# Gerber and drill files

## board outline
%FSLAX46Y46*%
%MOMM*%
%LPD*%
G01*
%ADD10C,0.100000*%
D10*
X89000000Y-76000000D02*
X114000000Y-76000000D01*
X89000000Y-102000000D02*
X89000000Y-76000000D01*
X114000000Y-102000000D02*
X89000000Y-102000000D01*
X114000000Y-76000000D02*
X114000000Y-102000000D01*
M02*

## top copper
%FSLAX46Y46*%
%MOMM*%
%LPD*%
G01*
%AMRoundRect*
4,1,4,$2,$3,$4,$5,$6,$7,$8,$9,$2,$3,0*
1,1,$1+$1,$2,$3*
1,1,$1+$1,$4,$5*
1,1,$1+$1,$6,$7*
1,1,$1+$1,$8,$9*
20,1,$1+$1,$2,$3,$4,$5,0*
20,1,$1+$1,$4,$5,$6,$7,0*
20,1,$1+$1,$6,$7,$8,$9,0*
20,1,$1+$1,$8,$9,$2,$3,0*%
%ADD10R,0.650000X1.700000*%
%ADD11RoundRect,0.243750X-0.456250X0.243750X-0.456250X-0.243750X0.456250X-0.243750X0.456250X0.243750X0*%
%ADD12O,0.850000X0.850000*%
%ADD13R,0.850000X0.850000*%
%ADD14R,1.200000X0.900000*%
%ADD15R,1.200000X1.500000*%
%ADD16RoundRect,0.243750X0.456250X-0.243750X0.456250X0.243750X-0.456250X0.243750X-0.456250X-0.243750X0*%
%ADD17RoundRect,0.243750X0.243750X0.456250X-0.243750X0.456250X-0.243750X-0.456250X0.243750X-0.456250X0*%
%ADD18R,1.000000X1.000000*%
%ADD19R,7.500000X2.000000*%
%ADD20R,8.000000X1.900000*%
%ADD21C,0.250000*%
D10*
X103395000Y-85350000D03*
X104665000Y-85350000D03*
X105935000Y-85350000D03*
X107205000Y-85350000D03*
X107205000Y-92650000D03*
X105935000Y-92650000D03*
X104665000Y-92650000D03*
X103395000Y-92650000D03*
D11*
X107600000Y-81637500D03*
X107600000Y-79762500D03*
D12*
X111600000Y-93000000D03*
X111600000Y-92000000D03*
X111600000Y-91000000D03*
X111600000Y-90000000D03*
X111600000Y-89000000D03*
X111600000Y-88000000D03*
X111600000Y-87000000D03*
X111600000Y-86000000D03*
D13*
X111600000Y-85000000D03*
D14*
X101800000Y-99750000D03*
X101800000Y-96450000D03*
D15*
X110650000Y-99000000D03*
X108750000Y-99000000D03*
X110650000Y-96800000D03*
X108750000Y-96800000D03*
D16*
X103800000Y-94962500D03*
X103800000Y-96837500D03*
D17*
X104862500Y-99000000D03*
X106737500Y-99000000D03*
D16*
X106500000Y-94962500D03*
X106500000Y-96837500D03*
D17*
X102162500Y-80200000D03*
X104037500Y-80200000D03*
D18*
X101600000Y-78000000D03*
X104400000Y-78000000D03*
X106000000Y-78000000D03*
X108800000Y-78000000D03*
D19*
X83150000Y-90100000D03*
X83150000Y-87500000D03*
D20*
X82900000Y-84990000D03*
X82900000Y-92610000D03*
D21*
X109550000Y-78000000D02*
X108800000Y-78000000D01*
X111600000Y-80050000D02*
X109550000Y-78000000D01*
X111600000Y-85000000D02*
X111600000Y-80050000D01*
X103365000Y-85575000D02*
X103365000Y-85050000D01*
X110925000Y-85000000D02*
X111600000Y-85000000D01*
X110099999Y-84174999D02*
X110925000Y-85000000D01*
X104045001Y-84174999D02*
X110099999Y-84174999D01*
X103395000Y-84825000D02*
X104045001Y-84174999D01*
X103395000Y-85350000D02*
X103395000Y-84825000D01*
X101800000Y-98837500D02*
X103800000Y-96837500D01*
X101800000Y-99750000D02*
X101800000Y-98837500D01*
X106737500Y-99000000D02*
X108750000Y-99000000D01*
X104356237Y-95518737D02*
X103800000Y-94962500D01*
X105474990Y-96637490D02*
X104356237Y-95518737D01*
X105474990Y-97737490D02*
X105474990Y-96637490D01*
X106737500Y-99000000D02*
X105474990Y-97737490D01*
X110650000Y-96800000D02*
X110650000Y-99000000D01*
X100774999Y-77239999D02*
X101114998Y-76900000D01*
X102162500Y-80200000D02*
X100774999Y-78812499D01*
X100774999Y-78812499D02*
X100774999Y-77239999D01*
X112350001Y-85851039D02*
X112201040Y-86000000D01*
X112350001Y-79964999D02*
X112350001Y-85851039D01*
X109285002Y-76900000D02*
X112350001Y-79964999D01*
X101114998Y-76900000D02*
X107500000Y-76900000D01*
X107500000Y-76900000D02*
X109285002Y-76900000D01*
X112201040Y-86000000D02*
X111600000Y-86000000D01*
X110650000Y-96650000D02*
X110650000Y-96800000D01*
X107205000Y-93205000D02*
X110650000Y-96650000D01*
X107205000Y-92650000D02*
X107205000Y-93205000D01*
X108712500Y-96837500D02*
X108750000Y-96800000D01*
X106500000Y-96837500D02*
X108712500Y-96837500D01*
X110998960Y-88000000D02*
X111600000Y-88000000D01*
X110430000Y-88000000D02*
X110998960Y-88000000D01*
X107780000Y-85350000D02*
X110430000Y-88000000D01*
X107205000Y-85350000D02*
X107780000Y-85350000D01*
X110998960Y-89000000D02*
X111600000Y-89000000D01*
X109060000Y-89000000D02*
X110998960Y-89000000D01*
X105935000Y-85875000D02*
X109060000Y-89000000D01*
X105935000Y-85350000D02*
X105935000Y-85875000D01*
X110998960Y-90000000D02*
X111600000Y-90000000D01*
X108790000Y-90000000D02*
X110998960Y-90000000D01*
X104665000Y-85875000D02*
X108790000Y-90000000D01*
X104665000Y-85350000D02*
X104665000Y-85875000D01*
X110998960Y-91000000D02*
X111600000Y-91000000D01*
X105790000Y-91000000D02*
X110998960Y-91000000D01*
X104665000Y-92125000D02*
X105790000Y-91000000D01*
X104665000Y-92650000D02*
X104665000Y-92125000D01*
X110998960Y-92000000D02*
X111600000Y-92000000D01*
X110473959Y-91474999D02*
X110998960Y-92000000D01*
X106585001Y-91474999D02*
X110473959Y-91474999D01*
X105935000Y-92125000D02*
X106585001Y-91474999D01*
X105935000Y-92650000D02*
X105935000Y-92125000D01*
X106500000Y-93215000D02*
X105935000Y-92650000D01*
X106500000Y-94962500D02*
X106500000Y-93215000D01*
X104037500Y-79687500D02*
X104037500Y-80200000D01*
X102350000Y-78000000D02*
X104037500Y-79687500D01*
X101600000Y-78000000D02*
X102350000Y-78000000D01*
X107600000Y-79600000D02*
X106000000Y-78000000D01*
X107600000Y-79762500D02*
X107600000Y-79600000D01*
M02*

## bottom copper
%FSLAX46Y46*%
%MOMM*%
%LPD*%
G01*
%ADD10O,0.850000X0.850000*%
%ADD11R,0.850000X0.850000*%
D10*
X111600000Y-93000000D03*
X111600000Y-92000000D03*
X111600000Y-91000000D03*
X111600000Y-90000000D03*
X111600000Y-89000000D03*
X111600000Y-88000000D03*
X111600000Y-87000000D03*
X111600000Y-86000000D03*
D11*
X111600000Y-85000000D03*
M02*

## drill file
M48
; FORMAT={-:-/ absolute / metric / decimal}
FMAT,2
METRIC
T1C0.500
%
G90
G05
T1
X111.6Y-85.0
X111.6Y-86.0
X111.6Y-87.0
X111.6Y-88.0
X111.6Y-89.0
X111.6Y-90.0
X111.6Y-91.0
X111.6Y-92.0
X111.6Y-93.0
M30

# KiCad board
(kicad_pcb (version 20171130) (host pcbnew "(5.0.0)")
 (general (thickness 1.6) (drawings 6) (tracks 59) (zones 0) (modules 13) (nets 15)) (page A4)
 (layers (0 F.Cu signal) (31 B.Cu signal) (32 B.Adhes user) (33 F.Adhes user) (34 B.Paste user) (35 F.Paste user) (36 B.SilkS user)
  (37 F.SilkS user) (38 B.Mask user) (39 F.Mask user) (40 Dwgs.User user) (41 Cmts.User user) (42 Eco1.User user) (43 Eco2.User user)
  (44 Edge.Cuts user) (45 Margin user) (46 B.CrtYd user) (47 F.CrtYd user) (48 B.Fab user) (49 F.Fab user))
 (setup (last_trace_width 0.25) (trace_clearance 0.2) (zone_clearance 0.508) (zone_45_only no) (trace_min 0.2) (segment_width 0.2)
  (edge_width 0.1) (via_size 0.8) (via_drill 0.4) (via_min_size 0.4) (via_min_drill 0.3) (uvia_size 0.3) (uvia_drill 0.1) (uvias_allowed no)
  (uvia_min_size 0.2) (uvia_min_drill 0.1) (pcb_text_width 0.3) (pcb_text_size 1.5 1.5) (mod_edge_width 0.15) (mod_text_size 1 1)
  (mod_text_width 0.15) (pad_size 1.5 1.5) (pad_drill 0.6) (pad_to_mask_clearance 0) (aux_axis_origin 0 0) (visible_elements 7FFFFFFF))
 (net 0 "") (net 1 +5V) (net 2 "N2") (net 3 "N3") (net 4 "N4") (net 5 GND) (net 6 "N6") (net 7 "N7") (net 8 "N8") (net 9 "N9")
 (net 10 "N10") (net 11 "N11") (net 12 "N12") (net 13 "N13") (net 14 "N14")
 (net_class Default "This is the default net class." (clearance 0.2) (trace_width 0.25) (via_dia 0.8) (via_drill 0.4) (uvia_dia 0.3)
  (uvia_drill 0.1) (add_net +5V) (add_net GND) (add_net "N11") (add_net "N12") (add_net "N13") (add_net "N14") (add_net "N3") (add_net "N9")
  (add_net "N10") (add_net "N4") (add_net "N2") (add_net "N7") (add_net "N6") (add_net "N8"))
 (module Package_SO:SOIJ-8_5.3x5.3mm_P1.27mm (layer F.Cu) (at 105.3 89 90)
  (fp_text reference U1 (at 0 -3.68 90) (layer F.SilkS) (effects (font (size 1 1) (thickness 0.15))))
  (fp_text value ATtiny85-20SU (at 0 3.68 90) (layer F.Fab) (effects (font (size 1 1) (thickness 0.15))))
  (pad 8 smd rect (at 3.65 -1.905 90) (size 1.7 0.65) (layers F.Cu F.Paste F.Mask) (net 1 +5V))
  (pad 7 smd rect (at 3.65 -0.635 90) (size 1.7 0.65) (layers F.Cu F.Paste F.Mask) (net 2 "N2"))
  (pad 6 smd rect (at 3.65 0.635 90) (size 1.7 0.65) (layers F.Cu F.Paste F.Mask) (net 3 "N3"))
  (pad 5 smd rect (at 3.65 1.905 90) (size 1.7 0.65) (layers F.Cu F.Paste F.Mask) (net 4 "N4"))
  (pad 4 smd rect (at -3.65 1.905 90) (size 1.7 0.65) (layers F.Cu F.Paste F.Mask) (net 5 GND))
  (pad 3 smd rect (at -3.65 0.635 90) (size 1.7 0.65) (layers F.Cu F.Paste F.Mask) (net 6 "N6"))
  (pad 2 smd rect (at -3.65 -0.635 90) (size 1.7 0.65) (layers F.Cu F.Paste F.Mask) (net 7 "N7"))
  (pad 1 smd rect (at -3.65 -1.905 90) (size 1.7 0.65) (layers F.Cu F.Paste F.Mask) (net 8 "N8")))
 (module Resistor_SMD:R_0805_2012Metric (layer F.Cu) (at 107.6 80.7 270)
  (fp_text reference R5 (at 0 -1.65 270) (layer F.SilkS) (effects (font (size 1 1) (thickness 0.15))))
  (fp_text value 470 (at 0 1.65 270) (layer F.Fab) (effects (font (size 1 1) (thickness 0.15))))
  (pad 2 smd roundrect (at 0.9375 0 270) (size 0.975 1.4) (layers F.Cu F.Paste F.Mask) (roundrect_rratio 0.25) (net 5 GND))
  (pad 1 smd roundrect (at -0.9375 0 270) (size 0.975 1.4) (layers F.Cu F.Paste F.Mask) (roundrect_rratio 0.25) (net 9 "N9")))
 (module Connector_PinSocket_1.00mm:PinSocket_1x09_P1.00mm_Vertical (layer F.Cu) (at 111.6 85)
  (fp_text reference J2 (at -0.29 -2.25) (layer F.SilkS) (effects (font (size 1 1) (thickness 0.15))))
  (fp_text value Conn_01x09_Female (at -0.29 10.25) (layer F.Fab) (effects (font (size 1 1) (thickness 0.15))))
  (pad 9 thru_hole oval (at 0 8) (size 0.85 0.85) (drill 0.5) (layers *.Cu *.Mask) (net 8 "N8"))
  (pad 8 thru_hole oval (at 0 7) (size 0.85 0.85) (drill 0.5) (layers *.Cu *.Mask) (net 6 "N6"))
  (pad 7 thru_hole oval (at 0 6) (size 0.85 0.85) (drill 0.5) (layers *.Cu *.Mask) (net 7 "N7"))
  (pad 6 thru_hole oval (at 0 5) (size 0.85 0.85) (drill 0.5) (layers *.Cu *.Mask) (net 2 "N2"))
  (pad 5 thru_hole oval (at 0 4) (size 0.85 0.85) (drill 0.5) (layers *.Cu *.Mask) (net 3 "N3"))
  (pad 4 thru_hole oval (at 0 3) (size 0.85 0.85) (drill 0.5) (layers *.Cu *.Mask) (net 4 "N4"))
  (pad 3 thru_hole oval (at 0 2) (size 0.85 0.85) (drill 0.5) (layers *.Cu *.Mask) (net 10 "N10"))
  (pad 2 thru_hole oval (at 0 1) (size 0.85 0.85) (drill 0.5) (layers *.Cu *.Mask) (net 5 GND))
  (pad 1 thru_hole rect (at 0 0) (size 0.85 0.85) (drill 0.5) (layers *.Cu *.Mask) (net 1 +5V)))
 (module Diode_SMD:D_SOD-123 (layer F.Cu) (at 101.8 98.1 270)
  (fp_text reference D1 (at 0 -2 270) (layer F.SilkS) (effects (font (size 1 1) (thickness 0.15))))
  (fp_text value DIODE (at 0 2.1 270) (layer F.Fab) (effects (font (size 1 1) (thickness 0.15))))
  (pad 2 smd rect (at 1.65 0 270) (size 0.9 1.2) (layers F.Cu F.Paste F.Mask) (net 1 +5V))
  (pad 1 smd rect (at -1.65 0 270) (size 0.9 1.2) (layers F.Cu F.Paste F.Mask) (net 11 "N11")))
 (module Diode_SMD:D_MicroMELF (layer F.Cu) (at 109.7 99)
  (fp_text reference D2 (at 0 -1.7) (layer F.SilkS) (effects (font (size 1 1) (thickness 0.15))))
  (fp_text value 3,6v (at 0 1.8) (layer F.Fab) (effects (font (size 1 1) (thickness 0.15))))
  (pad 2 smd rect (at 0.95 0) (size 1.2 1.5) (layers F.Cu F.Paste F.Mask) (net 5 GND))
  (pad 1 smd rect (at -0.95 0) (size 1.2 1.5) (layers F.Cu F.Paste F.Mask) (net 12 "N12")))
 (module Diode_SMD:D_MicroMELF (layer F.Cu) (at 109.7 96.8)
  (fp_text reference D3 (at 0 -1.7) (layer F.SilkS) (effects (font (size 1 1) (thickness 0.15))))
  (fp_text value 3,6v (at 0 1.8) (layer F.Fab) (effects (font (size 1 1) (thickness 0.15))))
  (pad 2 smd rect (at 0.95 0) (size 1.2 1.5) (layers F.Cu F.Paste F.Mask) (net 5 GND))
  (pad 1 smd rect (at -0.95 0) (size 1.2 1.5) (layers F.Cu F.Paste F.Mask) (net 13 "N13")))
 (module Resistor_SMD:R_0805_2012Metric (layer F.Cu) (at 103.8 95.9 90)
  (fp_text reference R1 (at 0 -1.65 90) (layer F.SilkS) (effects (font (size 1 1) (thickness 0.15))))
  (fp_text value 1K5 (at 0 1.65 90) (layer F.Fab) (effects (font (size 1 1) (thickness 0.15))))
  (pad 2 smd roundrect (at 0.9375 0 90) (size 0.975 1.4) (layers F.Cu F.Paste F.Mask) (roundrect_rratio 0.25) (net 12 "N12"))
  (pad 1 smd roundrect (at -0.9375 0 90) (size 0.975 1.4) (layers F.Cu F.Paste F.Mask) (roundrect_rratio 0.25) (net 1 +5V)))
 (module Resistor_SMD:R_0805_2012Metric (layer F.Cu) (at 105.8 99 180)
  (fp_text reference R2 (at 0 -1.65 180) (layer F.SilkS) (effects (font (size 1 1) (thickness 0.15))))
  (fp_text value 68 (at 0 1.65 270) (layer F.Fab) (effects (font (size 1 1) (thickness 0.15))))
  (pad 2 smd roundrect (at 0.9375 0 180) (size 0.975 1.4) (layers F.Cu F.Paste F.Mask) (roundrect_rratio 0.25) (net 7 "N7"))
  (pad 1 smd roundrect (at -0.9375 0 180) (size 0.975 1.4) (layers F.Cu F.Paste F.Mask) (roundrect_rratio 0.25) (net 12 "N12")))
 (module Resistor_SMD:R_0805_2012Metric (layer F.Cu) (at 106.5 95.9 90)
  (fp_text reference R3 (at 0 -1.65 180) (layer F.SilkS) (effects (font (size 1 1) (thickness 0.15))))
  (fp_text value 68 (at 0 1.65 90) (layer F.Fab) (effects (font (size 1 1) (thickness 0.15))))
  (pad 2 smd roundrect (at 0.9375 0 90) (size 0.975 1.4) (layers F.Cu F.Paste F.Mask) (roundrect_rratio 0.25) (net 6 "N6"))
  (pad 1 smd roundrect (at -0.9375 0 90) (size 0.975 1.4) (layers F.Cu F.Paste F.Mask) (roundrect_rratio 0.25) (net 13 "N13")))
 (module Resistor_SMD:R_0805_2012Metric (layer F.Cu) (at 103.1 80.2 180)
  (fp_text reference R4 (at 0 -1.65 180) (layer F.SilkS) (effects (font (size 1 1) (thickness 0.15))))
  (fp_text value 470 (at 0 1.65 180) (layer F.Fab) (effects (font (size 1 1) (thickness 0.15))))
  (pad 2 smd roundrect (at 0.9375 0 180) (size 0.975 1.4) (layers F.Cu F.Paste F.Mask) (roundrect_rratio 0.25) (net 5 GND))
  (pad 1 smd roundrect (at -0.9375 0 180) (size 0.975 1.4) (layers F.Cu F.Paste F.Mask) (roundrect_rratio 0.25) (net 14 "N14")))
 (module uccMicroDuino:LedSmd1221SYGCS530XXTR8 (layer F.Cu) (at 103 78)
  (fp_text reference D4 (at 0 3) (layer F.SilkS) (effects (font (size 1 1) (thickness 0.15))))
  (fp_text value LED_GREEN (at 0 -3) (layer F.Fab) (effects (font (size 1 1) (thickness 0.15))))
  (pad 1 smd rect (at -1.4 0) (size 1 1) (layers F.Cu F.Paste F.Mask) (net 14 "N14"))
  (pad 2 smd rect (at 1.4 0) (size 1 1) (layers F.Cu F.Paste F.Mask) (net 3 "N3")))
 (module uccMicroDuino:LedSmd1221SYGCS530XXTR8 (layer F.Cu) (at 107.4 78)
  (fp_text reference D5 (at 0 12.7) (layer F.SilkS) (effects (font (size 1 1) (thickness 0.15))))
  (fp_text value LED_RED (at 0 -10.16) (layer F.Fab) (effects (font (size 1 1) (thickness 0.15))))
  (pad 1 smd rect (at -1.4 0) (size 1 1) (layers F.Cu F.Paste F.Mask) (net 9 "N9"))
  (pad 2 smd rect (at 1.4 0) (size 1 1) (layers F.Cu F.Paste F.Mask) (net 1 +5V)))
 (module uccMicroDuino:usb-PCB (layer F.Cu) (at 78 88.8 270)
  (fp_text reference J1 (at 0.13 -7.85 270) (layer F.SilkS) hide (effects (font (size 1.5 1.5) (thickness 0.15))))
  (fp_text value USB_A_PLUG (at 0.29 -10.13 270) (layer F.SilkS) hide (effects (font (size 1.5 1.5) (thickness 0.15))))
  (pad 2 connect rect (at 1.3 -5.15 270) (size 2 7.5) (layers F.Cu F.Mask) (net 12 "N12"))
  (pad 3 connect rect (at -1.3 -5.15 270) (size 2 7.5) (layers F.Cu F.Mask) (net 13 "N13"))
  (pad 4 connect rect (at -3.81 -4.9 270) (size 1.9 8) (layers F.Cu F.Mask) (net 5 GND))
  (pad 1 connect rect (at 3.81 -4.9 270) (size 1.9 8) (layers F.Cu F.Mask) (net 11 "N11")))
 (gr_line (start 89 76) (end 114 76) (layer Edge.Cuts) (width 0.1))
 (gr_line (start 89 102) (end 89 76) (layer Edge.Cuts) (width 0.1))
 (gr_line (start 114 102) (end 89 102) (layer Edge.Cuts) (width 0.1))
 (gr_line (start 114 76) (end 114 102) (layer Edge.Cuts) (width 0.1))
 (segment (start 109.55 78) (end 108.8 78) (width 0.25) (layer F.Cu) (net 1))
 (segment (start 111.6 80.05) (end 109.55 78) (width 0.25) (layer F.Cu) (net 1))
 (segment (start 111.6 85) (end 111.6 80.05) (width 0.25) (layer F.Cu) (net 1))
 (segment (start 103.365 85.575) (end 103.365 85.05) (width 0.25) (layer F.Cu) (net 1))
 (segment (start 110.925 85) (end 111.6 85) (width 0.25) (layer F.Cu) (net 1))
 (segment (start 110.099999 84.174999) (end 110.925 85) (width 0.25) (layer F.Cu) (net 1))
 (segment (start 104.045001 84.174999) (end 110.099999 84.174999) (width 0.25) (layer F.Cu) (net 1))
 (segment (start 103.395 84.825) (end 104.045001 84.174999) (width 0.25) (layer F.Cu) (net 1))
 (segment (start 103.395 85.35) (end 103.395 84.825) (width 0.25) (layer F.Cu) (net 1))
 (segment (start 101.8 98.8375) (end 103.8 96.8375) (width 0.25) (layer F.Cu) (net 1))
 (segment (start 101.8 99.75) (end 101.8 98.8375) (width 0.25) (layer F.Cu) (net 1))
 (segment (start 106.7375 99) (end 108.75 99) (width 0.25) (layer F.Cu) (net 12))
 (segment (start 104.356237 95.518737) (end 103.8 94.9625) (width 0.25) (layer F.Cu) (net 12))
 (segment (start 105.47499 96.63749) (end 104.356237 95.518737) (width 0.25) (layer F.Cu) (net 12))
 (segment (start 105.47499 97.73749) (end 105.47499 96.63749) (width 0.25) (layer F.Cu) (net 12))
 (segment (start 106.7375 99) (end 105.47499 97.73749) (width 0.25) (layer F.Cu) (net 12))
 (segment (start 110.65 96.8) (end 110.65 99) (width 0.25) (layer F.Cu) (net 5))
 (segment (start 100.774999 77.239999) (end 101.114998 76.9) (width 0.25) (layer F.Cu) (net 5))
 (segment (start 102.1625 80.2) (end 100.774999 78.812499) (width 0.25) (layer F.Cu) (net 5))
 (segment (start 100.774999 78.812499) (end 100.774999 77.239999) (width 0.25) (layer F.Cu) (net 5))
 (segment (start 112.350001 85.851039) (end 112.20104 86) (width 0.25) (layer F.Cu) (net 5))
 (segment (start 112.350001 79.964999) (end 112.350001 85.851039) (width 0.25) (layer F.Cu) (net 5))
 (segment (start 109.285002 76.9) (end 112.350001 79.964999) (width 0.25) (layer F.Cu) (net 5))
 (segment (start 101.114998 76.9) (end 107.5 76.9) (width 0.25) (layer F.Cu) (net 5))
 (segment (start 107.5 76.9) (end 109.285002 76.9) (width 0.25) (layer F.Cu) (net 5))
 (segment (start 112.20104 86) (end 111.6 86) (width 0.25) (layer F.Cu) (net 5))
 (segment (start 110.65 96.65) (end 110.65 96.8) (width 0.25) (layer F.Cu) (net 5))
 (segment (start 107.205 93.205) (end 110.65 96.65) (width 0.25) (layer F.Cu) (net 5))
 (segment (start 107.205 92.65) (end 107.205 93.205) (width 0.25) (layer F.Cu) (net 5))
 (segment (start 108.7125 96.8375) (end 108.75 96.8) (width 0.25) (layer F.Cu) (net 13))
 (segment (start 106.5 96.8375) (end 108.7125 96.8375) (width 0.25) (layer F.Cu) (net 13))
 (segment (start 110.99896 88) (end 111.6 88) (width 0.25) (layer F.Cu) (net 4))
 (segment (start 110.43 88) (end 110.99896 88) (width 0.25) (layer F.Cu) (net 4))
 (segment (start 107.78 85.35) (end 110.43 88) (width 0.25) (layer F.Cu) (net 4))
 (segment (start 107.205 85.35) (end 107.78 85.35) (width 0.25) (layer F.Cu) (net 4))
 (segment (start 110.99896 89) (end 111.6 89) (width 0.25) (layer F.Cu) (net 3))
 (segment (start 109.06 89) (end 110.99896 89) (width 0.25) (layer F.Cu) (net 3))
 (segment (start 105.935 85.875) (end 109.06 89) (width 0.25) (layer F.Cu) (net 3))
 (segment (start 105.935 85.35) (end 105.935 85.875) (width 0.25) (layer F.Cu) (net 3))
 (segment (start 110.99896 90) (end 111.6 90) (width 0.25) (layer F.Cu) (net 2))
 (segment (start 108.79 90) (end 110.99896 90) (width 0.25) (layer F.Cu) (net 2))
 (segment (start 104.665 85.875) (end 108.79 90) (width 0.25) (layer F.Cu) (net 2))
 (segment (start 104.665 85.35) (end 104.665 85.875) (width 0.25) (layer F.Cu) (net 2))
 (segment (start 110.99896 91) (end 111.6 91) (width 0.25) (layer F.Cu) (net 7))
 (segment (start 105.79 91) (end 110.99896 91) (width 0.25) (layer F.Cu) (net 7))
 (segment (start 104.665 92.125) (end 105.79 91) (width 0.25) (layer F.Cu) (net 7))
 (segment (start 104.665 92.65) (end 104.665 92.125) (width 0.25) (layer F.Cu) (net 7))
 (segment (start 110.99896 92) (end 111.6 92) (width 0.25) (layer F.Cu) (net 6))
 (segment (start 110.473959 91.474999) (end 110.99896 92) (width 0.25) (layer F.Cu) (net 6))
 (segment (start 106.585001 91.474999) (end 110.473959 91.474999) (width 0.25) (layer F.Cu) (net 6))
 (segment (start 105.935 92.125) (end 106.585001 91.474999) (width 0.25) (layer F.Cu) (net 6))
 (segment (start 105.935 92.65) (end 105.935 92.125) (width 0.25) (layer F.Cu) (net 6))
 (segment (start 106.5 93.215) (end 105.935 92.65) (width 0.25) (layer F.Cu) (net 6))
 (segment (start 106.5 94.9625) (end 106.5 93.215) (width 0.25) (layer F.Cu) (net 6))
 (segment (start 104.0375 79.6875) (end 104.0375 80.2) (width 0.25) (layer F.Cu) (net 14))
 (segment (start 102.35 78) (end 104.0375 79.6875) (width 0.25) (layer F.Cu) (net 14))
 (segment (start 101.6 78) (end 102.35 78) (width 0.25) (layer F.Cu) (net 14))
 (segment (start 107.6 79.6) (end 106 78) (width 0.25) (layer F.Cu) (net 9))
 (segment (start 107.6 79.7625) (end 107.6 79.6) (width 0.25) (layer F.Cu) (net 9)))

